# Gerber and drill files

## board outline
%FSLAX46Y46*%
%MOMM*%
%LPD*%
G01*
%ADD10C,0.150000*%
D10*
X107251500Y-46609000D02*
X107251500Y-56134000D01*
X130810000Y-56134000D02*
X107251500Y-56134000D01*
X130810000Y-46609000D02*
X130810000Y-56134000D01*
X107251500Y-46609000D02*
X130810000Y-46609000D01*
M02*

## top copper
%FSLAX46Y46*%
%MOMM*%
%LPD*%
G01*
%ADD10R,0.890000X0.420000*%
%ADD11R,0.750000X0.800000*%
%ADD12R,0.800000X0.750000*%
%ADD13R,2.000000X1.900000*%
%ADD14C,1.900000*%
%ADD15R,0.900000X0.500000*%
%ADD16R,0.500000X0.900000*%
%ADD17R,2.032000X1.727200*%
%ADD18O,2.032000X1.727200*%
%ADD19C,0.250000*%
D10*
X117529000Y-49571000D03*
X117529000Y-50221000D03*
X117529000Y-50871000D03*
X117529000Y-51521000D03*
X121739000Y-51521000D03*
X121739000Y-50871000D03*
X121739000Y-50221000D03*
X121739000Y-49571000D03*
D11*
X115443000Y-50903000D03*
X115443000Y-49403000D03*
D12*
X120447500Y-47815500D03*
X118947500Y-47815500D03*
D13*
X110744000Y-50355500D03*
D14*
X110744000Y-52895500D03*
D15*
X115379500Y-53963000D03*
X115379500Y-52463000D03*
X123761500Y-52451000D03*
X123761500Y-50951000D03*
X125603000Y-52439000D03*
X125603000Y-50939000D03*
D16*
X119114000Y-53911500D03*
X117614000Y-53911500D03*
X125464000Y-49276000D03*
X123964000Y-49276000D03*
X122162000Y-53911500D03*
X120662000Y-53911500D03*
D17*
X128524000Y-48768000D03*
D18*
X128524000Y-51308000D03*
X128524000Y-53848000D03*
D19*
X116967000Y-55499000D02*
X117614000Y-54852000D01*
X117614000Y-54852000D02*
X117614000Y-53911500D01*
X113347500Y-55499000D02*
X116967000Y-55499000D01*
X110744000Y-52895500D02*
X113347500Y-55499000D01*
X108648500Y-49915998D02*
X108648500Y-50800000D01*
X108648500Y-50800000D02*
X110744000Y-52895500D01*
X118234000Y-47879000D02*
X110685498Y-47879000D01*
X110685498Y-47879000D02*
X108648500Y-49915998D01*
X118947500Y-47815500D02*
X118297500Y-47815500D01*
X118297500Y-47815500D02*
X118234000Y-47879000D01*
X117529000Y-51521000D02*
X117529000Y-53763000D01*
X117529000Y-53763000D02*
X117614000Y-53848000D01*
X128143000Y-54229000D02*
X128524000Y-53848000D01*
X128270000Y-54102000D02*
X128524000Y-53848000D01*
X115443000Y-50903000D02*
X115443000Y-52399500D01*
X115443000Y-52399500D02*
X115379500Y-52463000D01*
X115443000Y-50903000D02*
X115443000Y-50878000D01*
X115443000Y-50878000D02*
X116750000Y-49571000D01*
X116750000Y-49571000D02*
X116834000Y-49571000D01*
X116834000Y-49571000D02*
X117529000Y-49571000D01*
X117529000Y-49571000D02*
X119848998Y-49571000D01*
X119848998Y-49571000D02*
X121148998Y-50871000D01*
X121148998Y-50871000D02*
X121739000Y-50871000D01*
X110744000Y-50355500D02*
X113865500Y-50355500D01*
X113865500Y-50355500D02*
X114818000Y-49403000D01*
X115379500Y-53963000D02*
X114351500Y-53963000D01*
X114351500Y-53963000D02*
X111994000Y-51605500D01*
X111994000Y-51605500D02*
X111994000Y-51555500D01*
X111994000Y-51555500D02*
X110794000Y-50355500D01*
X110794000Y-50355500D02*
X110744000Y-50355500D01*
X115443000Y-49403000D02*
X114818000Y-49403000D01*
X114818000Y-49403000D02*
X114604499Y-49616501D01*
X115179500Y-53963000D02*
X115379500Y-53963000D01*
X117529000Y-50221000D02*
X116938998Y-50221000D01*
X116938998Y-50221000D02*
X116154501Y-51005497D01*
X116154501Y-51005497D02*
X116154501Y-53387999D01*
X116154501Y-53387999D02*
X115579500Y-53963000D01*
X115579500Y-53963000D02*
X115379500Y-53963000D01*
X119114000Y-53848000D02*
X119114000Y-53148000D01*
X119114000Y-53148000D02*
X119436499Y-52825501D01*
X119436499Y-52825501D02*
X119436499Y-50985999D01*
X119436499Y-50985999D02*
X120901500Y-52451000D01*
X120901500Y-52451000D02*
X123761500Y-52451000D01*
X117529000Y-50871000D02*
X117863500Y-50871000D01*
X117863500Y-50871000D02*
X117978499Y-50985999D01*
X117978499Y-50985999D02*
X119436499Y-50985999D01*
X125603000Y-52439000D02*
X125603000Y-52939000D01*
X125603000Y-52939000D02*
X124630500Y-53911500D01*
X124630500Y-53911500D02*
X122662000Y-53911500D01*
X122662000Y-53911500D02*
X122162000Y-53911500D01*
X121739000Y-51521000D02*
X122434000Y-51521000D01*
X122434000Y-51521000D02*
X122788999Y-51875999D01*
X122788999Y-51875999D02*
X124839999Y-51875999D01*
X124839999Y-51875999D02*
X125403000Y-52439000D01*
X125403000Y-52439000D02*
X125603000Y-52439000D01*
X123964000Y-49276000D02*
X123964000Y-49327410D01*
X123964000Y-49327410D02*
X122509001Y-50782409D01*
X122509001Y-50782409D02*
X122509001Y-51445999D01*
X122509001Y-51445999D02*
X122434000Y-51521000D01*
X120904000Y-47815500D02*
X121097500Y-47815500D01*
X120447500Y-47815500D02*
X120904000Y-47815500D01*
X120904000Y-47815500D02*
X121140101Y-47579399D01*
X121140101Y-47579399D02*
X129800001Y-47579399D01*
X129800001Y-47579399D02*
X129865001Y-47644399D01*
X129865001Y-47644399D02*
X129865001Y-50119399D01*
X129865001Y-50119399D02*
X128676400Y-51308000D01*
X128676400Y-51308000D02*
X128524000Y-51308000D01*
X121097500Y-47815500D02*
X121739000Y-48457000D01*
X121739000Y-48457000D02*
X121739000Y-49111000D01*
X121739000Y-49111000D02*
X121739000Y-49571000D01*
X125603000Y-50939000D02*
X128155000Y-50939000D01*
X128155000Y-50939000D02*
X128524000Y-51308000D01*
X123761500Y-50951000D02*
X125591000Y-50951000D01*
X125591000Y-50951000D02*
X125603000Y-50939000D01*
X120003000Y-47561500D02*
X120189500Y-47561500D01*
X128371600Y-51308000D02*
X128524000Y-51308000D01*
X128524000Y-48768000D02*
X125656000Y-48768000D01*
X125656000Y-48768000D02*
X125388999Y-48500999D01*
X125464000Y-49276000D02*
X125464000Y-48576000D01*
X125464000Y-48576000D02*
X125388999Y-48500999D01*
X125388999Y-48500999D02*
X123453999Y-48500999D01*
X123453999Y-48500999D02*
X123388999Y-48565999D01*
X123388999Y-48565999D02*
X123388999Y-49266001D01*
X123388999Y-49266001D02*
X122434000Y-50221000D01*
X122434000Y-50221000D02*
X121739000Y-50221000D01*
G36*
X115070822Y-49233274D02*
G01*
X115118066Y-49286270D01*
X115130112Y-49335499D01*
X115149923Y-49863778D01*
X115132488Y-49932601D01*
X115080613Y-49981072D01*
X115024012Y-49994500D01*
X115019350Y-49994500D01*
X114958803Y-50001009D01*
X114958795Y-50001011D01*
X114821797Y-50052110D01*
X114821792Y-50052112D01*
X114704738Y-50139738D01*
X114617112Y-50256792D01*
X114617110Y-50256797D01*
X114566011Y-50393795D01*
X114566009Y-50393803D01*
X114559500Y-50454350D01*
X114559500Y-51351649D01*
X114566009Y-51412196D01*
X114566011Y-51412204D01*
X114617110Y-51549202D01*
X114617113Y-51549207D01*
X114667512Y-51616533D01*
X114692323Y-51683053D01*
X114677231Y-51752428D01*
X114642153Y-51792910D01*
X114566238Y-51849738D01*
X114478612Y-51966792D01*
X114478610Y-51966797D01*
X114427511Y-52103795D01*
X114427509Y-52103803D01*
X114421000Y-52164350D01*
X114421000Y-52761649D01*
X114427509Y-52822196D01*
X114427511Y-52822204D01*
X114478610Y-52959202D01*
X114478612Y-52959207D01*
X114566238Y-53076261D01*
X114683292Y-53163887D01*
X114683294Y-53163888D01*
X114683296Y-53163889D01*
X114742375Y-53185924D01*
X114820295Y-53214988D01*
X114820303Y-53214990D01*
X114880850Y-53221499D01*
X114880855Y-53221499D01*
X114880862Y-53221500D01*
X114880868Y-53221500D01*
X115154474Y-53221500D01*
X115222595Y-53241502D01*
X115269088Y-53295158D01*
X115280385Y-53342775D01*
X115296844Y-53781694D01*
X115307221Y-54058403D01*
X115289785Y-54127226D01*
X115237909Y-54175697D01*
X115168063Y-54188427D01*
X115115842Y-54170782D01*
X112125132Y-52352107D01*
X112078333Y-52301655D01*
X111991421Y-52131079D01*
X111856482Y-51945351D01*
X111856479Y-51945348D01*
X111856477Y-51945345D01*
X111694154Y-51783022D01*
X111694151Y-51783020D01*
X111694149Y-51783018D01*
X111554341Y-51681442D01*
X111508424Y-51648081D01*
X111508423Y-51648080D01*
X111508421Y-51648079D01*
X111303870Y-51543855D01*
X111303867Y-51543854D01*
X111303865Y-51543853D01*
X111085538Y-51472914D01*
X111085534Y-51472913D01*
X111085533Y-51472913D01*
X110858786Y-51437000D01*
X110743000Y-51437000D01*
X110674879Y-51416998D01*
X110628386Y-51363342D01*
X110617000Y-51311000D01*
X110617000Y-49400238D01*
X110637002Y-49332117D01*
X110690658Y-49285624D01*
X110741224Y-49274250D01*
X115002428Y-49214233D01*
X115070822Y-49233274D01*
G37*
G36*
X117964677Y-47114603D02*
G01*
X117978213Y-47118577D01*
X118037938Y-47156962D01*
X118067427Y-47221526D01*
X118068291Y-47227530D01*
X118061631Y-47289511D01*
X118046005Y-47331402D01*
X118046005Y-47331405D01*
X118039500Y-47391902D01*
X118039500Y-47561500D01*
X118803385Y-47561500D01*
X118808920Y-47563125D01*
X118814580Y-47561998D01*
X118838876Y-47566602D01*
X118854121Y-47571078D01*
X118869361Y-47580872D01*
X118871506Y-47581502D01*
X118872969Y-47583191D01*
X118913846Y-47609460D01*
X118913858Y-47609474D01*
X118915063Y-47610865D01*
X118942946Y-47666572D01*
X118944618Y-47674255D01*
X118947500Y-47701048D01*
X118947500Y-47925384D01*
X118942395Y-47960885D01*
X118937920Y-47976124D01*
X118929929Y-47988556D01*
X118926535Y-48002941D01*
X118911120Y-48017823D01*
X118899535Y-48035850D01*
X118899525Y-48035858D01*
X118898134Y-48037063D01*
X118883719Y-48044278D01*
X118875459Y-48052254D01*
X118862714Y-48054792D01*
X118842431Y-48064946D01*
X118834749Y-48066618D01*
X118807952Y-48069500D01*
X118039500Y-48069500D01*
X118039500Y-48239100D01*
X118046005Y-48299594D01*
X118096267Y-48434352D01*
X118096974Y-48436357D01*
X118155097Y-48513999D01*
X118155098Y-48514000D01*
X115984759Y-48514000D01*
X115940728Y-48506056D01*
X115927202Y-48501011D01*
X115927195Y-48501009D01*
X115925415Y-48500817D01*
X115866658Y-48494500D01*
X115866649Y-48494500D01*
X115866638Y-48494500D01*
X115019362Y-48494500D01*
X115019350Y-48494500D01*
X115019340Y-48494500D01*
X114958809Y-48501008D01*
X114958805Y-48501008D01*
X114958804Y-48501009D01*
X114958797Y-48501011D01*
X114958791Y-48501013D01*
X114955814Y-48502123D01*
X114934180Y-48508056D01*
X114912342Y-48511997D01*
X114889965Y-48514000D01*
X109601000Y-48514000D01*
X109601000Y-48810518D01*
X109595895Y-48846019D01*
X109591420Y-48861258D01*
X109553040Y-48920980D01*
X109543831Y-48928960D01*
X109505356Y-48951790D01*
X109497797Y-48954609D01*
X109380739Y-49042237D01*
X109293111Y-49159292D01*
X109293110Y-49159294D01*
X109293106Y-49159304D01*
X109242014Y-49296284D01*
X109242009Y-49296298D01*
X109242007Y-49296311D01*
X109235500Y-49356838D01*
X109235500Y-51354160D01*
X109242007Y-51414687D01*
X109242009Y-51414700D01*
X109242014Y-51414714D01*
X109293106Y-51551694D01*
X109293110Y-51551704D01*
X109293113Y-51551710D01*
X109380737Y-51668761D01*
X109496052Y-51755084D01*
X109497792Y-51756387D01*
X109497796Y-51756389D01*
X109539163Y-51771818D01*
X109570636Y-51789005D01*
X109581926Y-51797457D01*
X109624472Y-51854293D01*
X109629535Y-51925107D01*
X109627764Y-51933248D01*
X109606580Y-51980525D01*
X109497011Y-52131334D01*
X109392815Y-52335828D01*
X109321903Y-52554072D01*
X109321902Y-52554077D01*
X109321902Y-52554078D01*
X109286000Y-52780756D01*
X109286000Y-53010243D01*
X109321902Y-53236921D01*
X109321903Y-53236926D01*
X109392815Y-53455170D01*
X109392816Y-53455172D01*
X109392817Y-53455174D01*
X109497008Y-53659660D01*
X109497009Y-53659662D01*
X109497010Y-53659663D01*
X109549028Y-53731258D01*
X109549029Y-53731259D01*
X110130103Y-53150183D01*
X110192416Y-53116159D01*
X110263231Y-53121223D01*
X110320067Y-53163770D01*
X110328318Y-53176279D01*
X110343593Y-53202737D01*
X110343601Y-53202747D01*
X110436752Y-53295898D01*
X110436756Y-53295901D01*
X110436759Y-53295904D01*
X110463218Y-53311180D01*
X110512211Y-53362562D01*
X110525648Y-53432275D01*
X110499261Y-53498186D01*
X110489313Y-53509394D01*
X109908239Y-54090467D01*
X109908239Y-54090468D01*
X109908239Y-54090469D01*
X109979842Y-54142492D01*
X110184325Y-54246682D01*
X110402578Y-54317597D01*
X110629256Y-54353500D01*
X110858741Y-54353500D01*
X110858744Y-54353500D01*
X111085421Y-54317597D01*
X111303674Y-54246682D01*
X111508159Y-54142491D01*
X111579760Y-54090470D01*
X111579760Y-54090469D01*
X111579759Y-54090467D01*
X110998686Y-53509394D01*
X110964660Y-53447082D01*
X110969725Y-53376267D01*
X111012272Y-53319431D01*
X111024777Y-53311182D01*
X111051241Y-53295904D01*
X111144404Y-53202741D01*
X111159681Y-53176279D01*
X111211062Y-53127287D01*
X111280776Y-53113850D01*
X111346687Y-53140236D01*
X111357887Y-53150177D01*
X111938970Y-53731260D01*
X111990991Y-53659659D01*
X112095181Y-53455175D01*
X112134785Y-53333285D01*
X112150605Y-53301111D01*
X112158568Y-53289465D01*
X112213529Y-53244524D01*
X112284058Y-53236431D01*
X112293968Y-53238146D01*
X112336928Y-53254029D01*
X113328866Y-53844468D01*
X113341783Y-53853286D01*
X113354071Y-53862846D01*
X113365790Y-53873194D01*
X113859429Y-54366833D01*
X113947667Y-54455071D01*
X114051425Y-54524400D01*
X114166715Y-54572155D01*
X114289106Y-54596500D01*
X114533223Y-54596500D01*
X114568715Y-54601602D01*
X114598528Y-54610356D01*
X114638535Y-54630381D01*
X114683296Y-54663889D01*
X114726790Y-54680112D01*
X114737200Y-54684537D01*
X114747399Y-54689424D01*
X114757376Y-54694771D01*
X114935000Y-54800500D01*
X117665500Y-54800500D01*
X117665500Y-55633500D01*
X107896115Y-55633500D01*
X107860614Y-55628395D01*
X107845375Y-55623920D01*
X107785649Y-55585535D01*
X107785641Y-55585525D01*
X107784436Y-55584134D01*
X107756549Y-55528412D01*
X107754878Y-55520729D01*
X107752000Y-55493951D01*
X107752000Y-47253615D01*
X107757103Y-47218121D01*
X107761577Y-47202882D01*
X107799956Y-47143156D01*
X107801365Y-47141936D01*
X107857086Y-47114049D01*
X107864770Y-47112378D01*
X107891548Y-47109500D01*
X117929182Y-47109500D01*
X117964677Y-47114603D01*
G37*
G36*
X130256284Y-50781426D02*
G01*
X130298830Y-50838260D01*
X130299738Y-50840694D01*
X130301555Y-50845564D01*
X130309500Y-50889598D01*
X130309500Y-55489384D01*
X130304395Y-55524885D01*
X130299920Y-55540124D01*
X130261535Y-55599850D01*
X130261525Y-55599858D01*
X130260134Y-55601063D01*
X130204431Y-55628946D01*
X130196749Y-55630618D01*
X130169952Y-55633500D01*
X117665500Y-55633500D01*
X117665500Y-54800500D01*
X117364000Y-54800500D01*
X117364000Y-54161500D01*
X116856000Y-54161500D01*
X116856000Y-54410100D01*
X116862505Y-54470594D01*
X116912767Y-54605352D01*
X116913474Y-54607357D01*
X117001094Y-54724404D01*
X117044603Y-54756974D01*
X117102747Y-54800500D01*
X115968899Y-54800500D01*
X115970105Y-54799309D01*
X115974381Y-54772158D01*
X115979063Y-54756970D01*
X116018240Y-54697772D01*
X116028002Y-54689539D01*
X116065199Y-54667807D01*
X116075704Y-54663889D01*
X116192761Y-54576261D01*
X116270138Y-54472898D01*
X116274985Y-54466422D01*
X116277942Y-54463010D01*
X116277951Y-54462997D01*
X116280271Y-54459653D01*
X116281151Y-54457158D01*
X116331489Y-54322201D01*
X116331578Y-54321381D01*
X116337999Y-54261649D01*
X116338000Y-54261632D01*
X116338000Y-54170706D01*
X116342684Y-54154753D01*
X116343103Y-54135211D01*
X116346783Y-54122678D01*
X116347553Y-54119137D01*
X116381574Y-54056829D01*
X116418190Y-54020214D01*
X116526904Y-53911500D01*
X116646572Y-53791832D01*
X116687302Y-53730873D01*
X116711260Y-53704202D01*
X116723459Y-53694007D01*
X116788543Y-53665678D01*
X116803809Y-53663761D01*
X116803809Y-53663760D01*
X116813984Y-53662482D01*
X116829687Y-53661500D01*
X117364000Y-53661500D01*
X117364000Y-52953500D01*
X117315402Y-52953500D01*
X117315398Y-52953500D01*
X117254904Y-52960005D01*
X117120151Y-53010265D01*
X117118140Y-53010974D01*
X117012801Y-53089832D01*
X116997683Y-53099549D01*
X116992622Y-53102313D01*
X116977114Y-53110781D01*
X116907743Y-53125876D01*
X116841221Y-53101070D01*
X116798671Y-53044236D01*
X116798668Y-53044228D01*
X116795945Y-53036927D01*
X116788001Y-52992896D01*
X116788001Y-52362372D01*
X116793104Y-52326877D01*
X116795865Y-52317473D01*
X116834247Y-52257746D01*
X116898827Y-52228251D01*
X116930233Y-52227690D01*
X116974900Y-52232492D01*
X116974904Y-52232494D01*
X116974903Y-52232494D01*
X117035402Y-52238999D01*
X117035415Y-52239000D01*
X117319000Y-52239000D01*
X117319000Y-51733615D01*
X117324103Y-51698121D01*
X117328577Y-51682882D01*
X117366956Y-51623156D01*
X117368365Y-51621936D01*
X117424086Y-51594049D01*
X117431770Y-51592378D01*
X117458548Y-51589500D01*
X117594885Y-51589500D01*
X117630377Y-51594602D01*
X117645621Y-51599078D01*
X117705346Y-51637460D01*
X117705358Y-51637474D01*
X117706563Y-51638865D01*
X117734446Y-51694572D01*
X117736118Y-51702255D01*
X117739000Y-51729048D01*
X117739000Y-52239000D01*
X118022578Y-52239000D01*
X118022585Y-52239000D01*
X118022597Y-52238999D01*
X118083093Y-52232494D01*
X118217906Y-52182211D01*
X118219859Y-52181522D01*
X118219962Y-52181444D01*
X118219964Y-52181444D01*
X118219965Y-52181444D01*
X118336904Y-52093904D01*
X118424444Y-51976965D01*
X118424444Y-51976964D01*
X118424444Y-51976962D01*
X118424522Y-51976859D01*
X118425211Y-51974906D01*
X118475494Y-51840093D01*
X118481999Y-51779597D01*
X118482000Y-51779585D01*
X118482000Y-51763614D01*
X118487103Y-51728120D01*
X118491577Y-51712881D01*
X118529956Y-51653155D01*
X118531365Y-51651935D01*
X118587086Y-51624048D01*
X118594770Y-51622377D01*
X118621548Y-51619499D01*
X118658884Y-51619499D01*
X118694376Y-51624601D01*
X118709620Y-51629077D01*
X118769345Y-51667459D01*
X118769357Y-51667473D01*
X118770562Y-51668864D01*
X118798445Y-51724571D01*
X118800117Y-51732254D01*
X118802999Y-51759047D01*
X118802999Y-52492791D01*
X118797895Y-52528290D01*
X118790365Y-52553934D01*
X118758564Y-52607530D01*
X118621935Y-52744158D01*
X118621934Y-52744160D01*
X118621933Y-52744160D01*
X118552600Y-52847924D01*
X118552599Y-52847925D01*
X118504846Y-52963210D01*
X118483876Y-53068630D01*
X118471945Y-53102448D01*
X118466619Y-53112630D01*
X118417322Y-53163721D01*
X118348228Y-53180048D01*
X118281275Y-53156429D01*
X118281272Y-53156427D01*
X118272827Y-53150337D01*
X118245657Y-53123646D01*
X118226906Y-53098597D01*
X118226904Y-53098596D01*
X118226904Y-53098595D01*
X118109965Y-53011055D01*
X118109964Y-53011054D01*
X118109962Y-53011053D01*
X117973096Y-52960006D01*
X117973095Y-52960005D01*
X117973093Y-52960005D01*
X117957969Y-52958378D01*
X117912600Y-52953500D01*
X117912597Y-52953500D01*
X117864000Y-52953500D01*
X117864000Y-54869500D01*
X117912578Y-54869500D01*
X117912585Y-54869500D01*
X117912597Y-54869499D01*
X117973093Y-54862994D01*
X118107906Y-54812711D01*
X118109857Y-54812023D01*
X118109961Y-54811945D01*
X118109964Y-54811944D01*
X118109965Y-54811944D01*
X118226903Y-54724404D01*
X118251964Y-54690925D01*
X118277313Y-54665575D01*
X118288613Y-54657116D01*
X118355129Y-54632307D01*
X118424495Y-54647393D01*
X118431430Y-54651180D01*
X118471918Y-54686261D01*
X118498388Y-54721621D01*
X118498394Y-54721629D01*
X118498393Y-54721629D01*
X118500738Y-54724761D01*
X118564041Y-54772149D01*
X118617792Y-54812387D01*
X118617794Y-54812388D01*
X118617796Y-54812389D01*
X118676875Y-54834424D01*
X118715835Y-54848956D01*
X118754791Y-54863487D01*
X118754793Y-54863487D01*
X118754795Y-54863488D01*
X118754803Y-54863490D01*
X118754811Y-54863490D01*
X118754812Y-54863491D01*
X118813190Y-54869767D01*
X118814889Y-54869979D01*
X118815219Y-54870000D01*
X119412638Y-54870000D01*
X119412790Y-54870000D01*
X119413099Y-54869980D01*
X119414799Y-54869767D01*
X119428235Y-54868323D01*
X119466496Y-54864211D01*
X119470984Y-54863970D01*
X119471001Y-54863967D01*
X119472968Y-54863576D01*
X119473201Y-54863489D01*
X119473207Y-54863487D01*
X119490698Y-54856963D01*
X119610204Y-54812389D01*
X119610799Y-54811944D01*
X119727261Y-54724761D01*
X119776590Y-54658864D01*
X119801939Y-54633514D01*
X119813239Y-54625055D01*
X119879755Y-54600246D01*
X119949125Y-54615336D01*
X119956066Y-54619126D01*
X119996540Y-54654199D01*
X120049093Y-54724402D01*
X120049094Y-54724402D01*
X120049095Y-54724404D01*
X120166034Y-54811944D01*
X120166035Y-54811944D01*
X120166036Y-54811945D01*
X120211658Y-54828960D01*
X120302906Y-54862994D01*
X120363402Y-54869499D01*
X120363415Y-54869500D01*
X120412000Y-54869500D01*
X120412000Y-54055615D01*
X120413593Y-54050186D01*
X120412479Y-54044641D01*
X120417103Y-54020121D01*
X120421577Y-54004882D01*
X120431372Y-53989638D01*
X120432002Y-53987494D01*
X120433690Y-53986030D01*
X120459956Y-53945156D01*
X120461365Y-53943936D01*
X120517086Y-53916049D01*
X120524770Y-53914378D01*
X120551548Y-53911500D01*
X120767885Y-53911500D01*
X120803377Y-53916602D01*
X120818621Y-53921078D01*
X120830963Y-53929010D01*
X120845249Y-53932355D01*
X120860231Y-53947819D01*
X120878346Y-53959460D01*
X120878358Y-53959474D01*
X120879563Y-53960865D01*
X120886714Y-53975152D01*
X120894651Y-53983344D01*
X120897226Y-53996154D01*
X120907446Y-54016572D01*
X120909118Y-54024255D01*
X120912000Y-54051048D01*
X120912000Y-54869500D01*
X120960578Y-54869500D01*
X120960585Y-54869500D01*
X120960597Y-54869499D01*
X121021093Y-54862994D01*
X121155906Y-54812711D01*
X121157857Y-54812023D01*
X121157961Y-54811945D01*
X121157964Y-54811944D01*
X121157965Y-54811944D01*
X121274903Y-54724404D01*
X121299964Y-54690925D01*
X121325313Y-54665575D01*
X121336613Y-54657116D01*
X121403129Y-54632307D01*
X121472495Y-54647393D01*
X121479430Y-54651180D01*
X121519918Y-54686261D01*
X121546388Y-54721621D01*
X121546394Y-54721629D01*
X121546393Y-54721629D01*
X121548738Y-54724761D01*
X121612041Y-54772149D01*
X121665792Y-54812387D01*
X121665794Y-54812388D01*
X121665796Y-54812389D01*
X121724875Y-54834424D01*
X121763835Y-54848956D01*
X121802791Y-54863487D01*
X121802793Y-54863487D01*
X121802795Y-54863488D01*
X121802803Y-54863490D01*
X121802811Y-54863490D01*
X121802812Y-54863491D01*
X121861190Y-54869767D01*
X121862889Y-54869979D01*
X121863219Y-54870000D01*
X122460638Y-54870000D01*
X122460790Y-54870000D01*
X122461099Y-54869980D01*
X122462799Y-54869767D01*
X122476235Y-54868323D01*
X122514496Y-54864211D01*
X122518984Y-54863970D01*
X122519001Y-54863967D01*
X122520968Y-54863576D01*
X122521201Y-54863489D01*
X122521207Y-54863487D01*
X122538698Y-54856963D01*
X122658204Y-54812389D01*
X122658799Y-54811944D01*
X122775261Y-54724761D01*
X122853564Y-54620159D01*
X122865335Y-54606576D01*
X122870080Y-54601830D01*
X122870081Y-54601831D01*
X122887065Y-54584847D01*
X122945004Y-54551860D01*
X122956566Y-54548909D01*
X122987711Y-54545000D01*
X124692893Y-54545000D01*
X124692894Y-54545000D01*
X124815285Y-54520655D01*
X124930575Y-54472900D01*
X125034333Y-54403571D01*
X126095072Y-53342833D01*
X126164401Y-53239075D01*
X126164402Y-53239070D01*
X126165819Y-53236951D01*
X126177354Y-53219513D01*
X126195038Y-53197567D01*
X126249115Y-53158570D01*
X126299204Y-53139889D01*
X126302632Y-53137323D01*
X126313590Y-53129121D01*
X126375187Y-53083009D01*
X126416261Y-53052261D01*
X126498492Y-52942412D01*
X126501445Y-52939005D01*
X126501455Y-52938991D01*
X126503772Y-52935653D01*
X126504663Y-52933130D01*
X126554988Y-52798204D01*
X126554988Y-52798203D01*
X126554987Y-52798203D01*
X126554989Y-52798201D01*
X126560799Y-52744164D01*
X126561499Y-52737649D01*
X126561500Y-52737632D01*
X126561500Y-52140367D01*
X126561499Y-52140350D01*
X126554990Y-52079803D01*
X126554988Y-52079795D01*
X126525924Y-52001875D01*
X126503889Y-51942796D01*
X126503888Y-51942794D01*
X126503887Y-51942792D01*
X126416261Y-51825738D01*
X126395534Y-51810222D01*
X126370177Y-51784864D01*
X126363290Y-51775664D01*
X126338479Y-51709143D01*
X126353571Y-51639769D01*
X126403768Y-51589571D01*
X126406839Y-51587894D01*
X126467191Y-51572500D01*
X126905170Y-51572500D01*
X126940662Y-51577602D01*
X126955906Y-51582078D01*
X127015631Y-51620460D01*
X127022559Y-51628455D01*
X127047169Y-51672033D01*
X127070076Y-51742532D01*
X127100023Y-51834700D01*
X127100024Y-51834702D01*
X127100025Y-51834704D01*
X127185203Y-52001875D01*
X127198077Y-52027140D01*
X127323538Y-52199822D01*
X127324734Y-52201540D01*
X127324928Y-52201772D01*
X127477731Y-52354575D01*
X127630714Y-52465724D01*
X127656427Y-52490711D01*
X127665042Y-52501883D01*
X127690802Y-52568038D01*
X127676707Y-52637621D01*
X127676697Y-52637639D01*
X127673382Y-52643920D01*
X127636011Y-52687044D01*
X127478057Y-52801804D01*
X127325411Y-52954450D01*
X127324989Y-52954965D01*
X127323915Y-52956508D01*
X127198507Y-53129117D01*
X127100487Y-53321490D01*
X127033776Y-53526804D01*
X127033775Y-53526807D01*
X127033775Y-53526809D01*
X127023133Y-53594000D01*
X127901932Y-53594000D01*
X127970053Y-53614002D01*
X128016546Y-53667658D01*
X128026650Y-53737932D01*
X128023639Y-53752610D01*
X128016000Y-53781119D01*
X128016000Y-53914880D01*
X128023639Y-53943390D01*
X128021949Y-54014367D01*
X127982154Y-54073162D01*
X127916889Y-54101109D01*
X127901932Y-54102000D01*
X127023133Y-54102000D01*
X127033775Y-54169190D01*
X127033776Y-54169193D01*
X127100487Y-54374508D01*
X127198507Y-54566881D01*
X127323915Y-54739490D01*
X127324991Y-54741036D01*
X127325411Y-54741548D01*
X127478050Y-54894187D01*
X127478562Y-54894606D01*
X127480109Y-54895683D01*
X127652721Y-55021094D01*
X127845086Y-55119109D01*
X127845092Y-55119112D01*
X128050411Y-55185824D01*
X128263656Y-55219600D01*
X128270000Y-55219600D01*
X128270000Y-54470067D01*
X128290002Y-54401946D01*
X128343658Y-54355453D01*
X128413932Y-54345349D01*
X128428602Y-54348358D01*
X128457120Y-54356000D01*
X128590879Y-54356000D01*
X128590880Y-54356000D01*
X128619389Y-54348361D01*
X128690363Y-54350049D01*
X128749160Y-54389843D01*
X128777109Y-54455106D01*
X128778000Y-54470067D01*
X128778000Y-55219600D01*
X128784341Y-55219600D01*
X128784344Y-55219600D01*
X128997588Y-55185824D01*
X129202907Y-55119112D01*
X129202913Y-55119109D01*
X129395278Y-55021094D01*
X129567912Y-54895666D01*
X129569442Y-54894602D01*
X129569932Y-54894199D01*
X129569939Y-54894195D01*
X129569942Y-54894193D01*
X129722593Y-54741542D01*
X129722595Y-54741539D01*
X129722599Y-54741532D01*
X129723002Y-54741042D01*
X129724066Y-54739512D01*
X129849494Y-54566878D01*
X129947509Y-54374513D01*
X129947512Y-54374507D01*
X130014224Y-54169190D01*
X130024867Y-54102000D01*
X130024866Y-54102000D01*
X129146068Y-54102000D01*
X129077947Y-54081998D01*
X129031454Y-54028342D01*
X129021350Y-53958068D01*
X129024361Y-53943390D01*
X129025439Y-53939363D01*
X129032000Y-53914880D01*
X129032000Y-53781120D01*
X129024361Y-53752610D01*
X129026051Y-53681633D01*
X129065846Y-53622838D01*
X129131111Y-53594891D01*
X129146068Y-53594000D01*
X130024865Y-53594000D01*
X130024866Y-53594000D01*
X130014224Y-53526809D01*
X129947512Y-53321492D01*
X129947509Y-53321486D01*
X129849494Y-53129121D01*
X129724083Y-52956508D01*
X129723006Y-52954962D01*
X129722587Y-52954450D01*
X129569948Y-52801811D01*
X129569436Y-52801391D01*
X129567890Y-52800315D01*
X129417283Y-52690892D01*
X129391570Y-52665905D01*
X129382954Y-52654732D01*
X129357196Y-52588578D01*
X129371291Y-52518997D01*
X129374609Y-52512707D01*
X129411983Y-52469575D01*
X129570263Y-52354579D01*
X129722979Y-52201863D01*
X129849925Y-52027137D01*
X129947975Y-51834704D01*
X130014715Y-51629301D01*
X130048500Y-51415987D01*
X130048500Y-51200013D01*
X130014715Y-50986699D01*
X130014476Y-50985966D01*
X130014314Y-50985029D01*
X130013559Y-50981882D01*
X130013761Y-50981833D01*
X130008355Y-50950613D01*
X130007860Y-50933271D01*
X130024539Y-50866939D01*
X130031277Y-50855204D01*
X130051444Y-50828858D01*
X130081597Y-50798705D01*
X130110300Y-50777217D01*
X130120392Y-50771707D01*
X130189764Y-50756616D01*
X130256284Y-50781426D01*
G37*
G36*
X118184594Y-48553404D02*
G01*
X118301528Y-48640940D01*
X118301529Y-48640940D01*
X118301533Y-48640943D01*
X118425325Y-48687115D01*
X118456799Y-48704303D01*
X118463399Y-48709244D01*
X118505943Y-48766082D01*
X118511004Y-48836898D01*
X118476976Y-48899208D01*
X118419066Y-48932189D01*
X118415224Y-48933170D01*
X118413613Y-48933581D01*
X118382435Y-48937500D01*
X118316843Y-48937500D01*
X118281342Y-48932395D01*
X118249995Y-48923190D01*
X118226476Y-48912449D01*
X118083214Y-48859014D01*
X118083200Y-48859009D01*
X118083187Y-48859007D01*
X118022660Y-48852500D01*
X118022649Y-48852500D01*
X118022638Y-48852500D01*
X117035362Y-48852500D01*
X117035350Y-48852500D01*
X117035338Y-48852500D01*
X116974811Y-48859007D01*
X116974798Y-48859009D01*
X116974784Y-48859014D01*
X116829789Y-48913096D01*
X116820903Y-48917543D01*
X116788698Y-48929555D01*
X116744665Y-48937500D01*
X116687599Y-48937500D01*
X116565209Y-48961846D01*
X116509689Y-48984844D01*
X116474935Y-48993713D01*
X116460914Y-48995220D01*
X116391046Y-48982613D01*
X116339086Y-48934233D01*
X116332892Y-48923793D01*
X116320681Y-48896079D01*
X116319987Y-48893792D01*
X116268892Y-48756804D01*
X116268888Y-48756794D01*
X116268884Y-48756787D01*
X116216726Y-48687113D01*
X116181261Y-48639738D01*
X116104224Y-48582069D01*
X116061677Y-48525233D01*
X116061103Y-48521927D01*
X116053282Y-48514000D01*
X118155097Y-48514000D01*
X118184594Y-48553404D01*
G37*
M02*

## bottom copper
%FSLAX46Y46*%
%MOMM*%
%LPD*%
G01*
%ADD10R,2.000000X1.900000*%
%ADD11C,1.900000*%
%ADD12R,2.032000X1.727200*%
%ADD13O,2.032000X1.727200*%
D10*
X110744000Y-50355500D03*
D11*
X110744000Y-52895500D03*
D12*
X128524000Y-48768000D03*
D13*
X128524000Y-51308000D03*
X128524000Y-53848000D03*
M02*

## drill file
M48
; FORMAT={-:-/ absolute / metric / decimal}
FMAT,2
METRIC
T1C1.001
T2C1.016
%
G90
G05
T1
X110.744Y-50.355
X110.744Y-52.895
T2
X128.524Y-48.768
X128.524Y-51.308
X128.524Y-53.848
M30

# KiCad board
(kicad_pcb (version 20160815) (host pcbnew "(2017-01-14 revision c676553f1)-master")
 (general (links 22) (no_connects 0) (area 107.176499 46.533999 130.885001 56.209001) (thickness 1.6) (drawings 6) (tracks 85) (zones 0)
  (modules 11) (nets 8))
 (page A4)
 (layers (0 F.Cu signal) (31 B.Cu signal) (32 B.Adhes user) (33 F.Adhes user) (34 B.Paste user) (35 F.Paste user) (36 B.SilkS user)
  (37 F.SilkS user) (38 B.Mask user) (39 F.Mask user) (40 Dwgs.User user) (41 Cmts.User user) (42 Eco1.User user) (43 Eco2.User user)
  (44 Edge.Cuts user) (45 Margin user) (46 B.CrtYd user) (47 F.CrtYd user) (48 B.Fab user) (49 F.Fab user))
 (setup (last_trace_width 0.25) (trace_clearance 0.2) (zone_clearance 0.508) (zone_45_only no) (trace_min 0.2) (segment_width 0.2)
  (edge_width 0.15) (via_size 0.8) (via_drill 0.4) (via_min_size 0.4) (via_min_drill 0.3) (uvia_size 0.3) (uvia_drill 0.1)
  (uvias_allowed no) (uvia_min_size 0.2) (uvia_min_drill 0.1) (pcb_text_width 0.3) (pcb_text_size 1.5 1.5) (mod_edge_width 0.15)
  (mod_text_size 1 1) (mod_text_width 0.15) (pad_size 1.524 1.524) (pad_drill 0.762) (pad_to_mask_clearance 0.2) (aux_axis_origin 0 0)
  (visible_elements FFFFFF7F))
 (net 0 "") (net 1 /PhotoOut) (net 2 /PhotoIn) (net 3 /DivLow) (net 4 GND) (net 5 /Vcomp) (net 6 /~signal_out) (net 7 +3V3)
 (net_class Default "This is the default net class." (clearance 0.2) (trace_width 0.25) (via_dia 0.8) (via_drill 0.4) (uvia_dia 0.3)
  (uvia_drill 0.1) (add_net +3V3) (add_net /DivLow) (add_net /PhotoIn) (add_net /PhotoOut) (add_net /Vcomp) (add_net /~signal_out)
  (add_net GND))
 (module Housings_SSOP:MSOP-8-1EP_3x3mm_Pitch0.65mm (layer F.Cu) (at 119.634 50.546)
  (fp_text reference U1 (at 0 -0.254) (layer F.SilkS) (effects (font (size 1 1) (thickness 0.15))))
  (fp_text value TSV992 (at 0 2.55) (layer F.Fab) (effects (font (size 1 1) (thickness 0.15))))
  (pad 1 smd rect (at -2.105 -0.975) (size 0.89 0.42) (layers F.Cu F.Paste F.Mask) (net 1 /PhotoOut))
  (pad 2 smd rect (at -2.105 -0.325) (size 0.89 0.42) (layers F.Cu F.Paste F.Mask) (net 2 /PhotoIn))
  (pad 3 smd rect (at -2.105 0.325) (size 0.89 0.42) (layers F.Cu F.Paste F.Mask) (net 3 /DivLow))
  (pad 4 smd rect (at -2.105 0.975) (size 0.89 0.42) (layers F.Cu F.Paste F.Mask) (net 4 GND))
  (pad 5 smd rect (at 2.105 0.975) (size 0.89 0.42) (layers F.Cu F.Paste F.Mask) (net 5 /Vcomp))
  (pad 6 smd rect (at 2.105 0.325) (size 0.89 0.42) (layers F.Cu F.Paste F.Mask) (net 1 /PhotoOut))
  (pad 7 smd rect (at 2.105 -0.325) (size 0.89 0.42) (layers F.Cu F.Paste F.Mask) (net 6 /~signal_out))
  (pad 8 smd rect (at 2.105 -0.975) (size 0.89 0.42) (layers F.Cu F.Paste F.Mask) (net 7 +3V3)))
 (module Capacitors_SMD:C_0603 (layer F.Cu) (at 115.443 50.153 90)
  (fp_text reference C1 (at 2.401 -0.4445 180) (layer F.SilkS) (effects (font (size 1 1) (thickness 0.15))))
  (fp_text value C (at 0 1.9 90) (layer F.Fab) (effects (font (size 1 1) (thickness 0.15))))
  (pad 1 smd rect (at -0.75 0 90) (size 0.8 0.75) (layers F.Cu F.Paste F.Mask) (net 1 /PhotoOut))
  (pad 2 smd rect (at 0.75 0 90) (size 0.8 0.75) (layers F.Cu F.Paste F.Mask) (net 2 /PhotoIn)))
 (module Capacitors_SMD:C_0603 (layer F.Cu) (at 119.6975 47.8155)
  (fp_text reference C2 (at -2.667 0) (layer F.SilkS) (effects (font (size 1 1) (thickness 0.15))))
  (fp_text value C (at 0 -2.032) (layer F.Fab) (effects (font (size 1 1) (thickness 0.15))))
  (pad 2 smd rect (at 0.75 0) (size 0.8 0.75) (layers F.Cu F.Paste F.Mask) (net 7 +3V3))
  (pad 1 smd rect (at -0.75 0) (size 0.8 0.75) (layers F.Cu F.Paste F.Mask) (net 4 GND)))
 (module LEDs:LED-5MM (layer F.Cu) (at 110.744 50.3555 270)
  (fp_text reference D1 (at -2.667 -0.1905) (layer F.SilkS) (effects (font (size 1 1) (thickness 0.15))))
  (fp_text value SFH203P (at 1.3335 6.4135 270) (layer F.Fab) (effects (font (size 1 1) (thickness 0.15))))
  (pad 1 thru_hole rect (at 0 0) (size 2 1.9) (drill 1.00076) (layers *.Cu *.Mask F.SilkS) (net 2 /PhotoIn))
  (pad 2 thru_hole circle (at 2.54 0 270) (size 1.9 1.9) (drill 1.00076) (layers *.Cu *.Mask F.SilkS) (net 4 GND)))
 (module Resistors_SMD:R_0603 (layer F.Cu) (at 115.3795 53.213 270)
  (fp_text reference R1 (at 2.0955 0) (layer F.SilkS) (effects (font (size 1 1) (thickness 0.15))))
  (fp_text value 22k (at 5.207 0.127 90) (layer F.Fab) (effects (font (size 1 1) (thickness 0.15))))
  (pad 2 smd rect (at 0.75 0 270) (size 0.5 0.9) (layers F.Cu F.Paste F.Mask) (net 2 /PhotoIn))
  (pad 1 smd rect (at -0.75 0 270) (size 0.5 0.9) (layers F.Cu F.Paste F.Mask) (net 1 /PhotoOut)))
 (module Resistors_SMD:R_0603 (layer F.Cu) (at 123.7615 51.701 270)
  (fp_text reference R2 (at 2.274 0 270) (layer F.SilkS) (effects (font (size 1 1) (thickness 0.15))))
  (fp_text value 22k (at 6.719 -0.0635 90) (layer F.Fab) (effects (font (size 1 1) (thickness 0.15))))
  (pad 2 smd rect (at 0.75 0 270) (size 0.5 0.9) (layers F.Cu F.Paste F.Mask) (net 3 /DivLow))
  (pad 1 smd rect (at -0.75 0 270) (size 0.5 0.9) (layers F.Cu F.Paste F.Mask) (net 7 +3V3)))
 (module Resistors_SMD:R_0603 (layer F.Cu) (at 125.603 51.689 270)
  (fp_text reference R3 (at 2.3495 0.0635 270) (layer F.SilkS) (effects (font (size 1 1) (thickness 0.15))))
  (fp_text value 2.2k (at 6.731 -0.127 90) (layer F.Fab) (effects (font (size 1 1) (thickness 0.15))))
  (pad 2 smd rect (at 0.75 0 270) (size 0.5 0.9) (layers F.Cu F.Paste F.Mask) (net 5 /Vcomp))
  (pad 1 smd rect (at -0.75 0 270) (size 0.5 0.9) (layers F.Cu F.Paste F.Mask) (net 7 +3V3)))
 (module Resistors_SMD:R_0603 (layer F.Cu) (at 118.364 53.9115 180)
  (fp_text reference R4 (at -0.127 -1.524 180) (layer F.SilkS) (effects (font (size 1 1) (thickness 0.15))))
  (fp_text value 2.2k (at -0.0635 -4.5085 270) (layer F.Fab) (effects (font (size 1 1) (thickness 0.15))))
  (pad 1 smd rect (at -0.75 0 180) (size 0.5 0.9) (layers F.Cu F.Paste F.Mask) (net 3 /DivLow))
  (pad 2 smd rect (at 0.75 0 180) (size 0.5 0.9) (layers F.Cu F.Paste F.Mask) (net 4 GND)))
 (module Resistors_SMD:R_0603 (layer F.Cu) (at 124.714 49.276 180)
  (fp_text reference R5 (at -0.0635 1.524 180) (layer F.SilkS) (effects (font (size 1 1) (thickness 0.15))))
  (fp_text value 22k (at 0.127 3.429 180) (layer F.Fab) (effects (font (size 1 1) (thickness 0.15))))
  (pad 1 smd rect (at -0.75 0 180) (size 0.5 0.9) (layers F.Cu F.Paste F.Mask) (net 6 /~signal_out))
  (pad 2 smd rect (at 0.75 0 180) (size 0.5 0.9) (layers F.Cu F.Paste F.Mask) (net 5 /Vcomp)))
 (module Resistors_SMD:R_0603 (layer F.Cu) (at 121.412 53.9115 180)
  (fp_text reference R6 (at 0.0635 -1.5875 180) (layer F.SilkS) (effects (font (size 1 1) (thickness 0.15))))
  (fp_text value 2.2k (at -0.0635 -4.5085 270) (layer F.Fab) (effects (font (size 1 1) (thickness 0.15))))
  (pad 1 smd rect (at -0.75 0 180) (size 0.5 0.9) (layers F.Cu F.Paste F.Mask) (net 5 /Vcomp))
  (pad 2 smd rect (at 0.75 0 180) (size 0.5 0.9) (layers F.Cu F.Paste F.Mask) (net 4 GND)))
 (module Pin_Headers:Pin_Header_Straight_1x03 (layer F.Cu) (at 128.524 48.768)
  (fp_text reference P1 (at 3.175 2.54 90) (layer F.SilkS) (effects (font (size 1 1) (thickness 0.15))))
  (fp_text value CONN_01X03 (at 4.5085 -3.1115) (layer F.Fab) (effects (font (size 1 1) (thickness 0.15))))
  (pad 1 thru_hole rect (at 0 0) (size 2.032 1.7272) (drill 1.016) (layers *.Cu *.Mask F.SilkS) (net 6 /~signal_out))
  (pad 2 thru_hole oval (at 0 2.54) (size 2.032 1.7272) (drill 1.016) (layers *.Cu *.Mask F.SilkS) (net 7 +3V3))
  (pad 3 thru_hole oval (at 0 5.08) (size 2.032 1.7272) (drill 1.016) (layers *.Cu *.Mask F.SilkS) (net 4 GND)))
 (gr_line (start 107.2515 46.609) (end 107.2515 56.134) (layer Edge.Cuts) (width 0.15))
 (gr_line (start 130.81 56.134) (end 107.2515 56.134) (layer Edge.Cuts) (width 0.15))
 (gr_line (start 130.81 46.609) (end 130.81 56.134) (layer Edge.Cuts) (width 0.15))
 (gr_line (start 107.2515 46.609) (end 130.81 46.609) (layer Edge.Cuts) (width 0.15))
 (segment (start 116.967 55.499) (end 117.614 54.852) (width 0.25) (layer F.Cu) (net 4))
 (segment (start 117.614 54.852) (end 117.614 53.9115) (width 0.25) (layer F.Cu) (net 4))
 (segment (start 113.3475 55.499) (end 116.967 55.499) (width 0.25) (layer F.Cu) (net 4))
 (segment (start 110.744 52.8955) (end 113.3475 55.499) (width 0.25) (layer F.Cu) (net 4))
 (segment (start 108.6485 49.915998) (end 108.6485 50.8) (width 0.25) (layer F.Cu) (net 4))
 (segment (start 108.6485 50.8) (end 110.744 52.8955) (width 0.25) (layer F.Cu) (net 4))
 (segment (start 118.234 47.879) (end 110.685498 47.879) (width 0.25) (layer F.Cu) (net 4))
 (segment (start 110.685498 47.879) (end 108.6485 49.915998) (width 0.25) (layer F.Cu) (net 4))
 (segment (start 118.9475 47.8155) (end 118.2975 47.8155) (width 0.25) (layer F.Cu) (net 4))
 (segment (start 118.2975 47.8155) (end 118.234 47.879) (width 0.25) (layer F.Cu) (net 4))
 (segment (start 117.529 51.521) (end 117.529 53.763) (width 0.25) (layer F.Cu) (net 4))
 (segment (start 117.529 53.763) (end 117.614 53.848) (width 0.25) (layer F.Cu) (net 4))
 (segment (start 128.143 54.229) (end 128.524 53.848) (width 0.25) (layer F.Cu) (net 4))
 (segment (start 128.27 54.102) (end 128.524 53.848) (width 0.25) (layer F.Cu) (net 4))
 (segment (start 115.443 50.903) (end 115.443 52.3995) (width 0.25) (layer F.Cu) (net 1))
 (segment (start 115.443 52.3995) (end 115.3795 52.463) (width 0.25) (layer F.Cu) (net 1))
 (segment (start 115.443 50.903) (end 115.443 50.878) (width 0.25) (layer F.Cu) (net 1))
 (segment (start 115.443 50.878) (end 116.75 49.571) (width 0.25) (layer F.Cu) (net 1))
 (segment (start 116.75 49.571) (end 116.834 49.571) (width 0.25) (layer F.Cu) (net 1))
 (segment (start 116.834 49.571) (end 117.529 49.571) (width 0.25) (layer F.Cu) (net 1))
 (segment (start 117.529 49.571) (end 119.848998 49.571) (width 0.25) (layer F.Cu) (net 1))
 (segment (start 119.848998 49.571) (end 121.148998 50.871) (width 0.25) (layer F.Cu) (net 1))
 (segment (start 121.148998 50.871) (end 121.739 50.871) (width 0.25) (layer F.Cu) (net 1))
 (segment (start 110.744 50.3555) (end 113.8655 50.3555) (width 0.25) (layer F.Cu) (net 2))
 (segment (start 113.8655 50.3555) (end 114.818 49.403) (width 0.25) (layer F.Cu) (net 2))
 (segment (start 115.3795 53.963) (end 114.3515 53.963) (width 0.25) (layer F.Cu) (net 2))
 (segment (start 114.3515 53.963) (end 111.994 51.6055) (width 0.25) (layer F.Cu) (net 2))
 (segment (start 111.994 51.6055) (end 111.994 51.5555) (width 0.25) (layer F.Cu) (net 2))
 (segment (start 111.994 51.5555) (end 110.794 50.3555) (width 0.25) (layer F.Cu) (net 2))
 (segment (start 110.794 50.3555) (end 110.744 50.3555) (width 0.25) (layer F.Cu) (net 2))
 (segment (start 115.443 49.403) (end 114.818 49.403) (width 0.25) (layer F.Cu) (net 2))
 (segment (start 114.818 49.403) (end 114.604499 49.616501) (width 0.25) (layer F.Cu) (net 2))
 (segment (start 115.1795 53.963) (end 115.3795 53.963) (width 0.25) (layer F.Cu) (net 2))
 (segment (start 117.529 50.221) (end 116.938998 50.221) (width 0.25) (layer F.Cu) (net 2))
 (segment (start 116.938998 50.221) (end 116.154501 51.005497) (width 0.25) (layer F.Cu) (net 2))
 (segment (start 116.154501 51.005497) (end 116.154501 53.387999) (width 0.25) (layer F.Cu) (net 2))
 (segment (start 116.154501 53.387999) (end 115.5795 53.963) (width 0.25) (layer F.Cu) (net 2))
 (segment (start 115.5795 53.963) (end 115.3795 53.963) (width 0.25) (layer F.Cu) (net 2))
 (segment (start 119.114 53.848) (end 119.114 53.148) (width 0.25) (layer F.Cu) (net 3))
 (segment (start 119.114 53.148) (end 119.436499 52.825501) (width 0.25) (layer F.Cu) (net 3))
 (segment (start 119.436499 52.825501) (end 119.436499 50.985999) (width 0.25) (layer F.Cu) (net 3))
 (segment (start 119.436499 50.985999) (end 120.9015 52.451) (width 0.25) (layer F.Cu) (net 3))
 (segment (start 120.9015 52.451) (end 123.7615 52.451) (width 0.25) (layer F.Cu) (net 3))
 (segment (start 117.529 50.871) (end 117.8635 50.871) (width 0.25) (layer F.Cu) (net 3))
 (segment (start 117.8635 50.871) (end 117.978499 50.985999) (width 0.25) (layer F.Cu) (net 3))
 (segment (start 117.978499 50.985999) (end 119.436499 50.985999) (width 0.25) (layer F.Cu) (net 3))
 (segment (start 125.603 52.439) (end 125.603 52.939) (width 0.25) (layer F.Cu) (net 5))
 (segment (start 125.603 52.939) (end 124.6305 53.9115) (width 0.25) (layer F.Cu) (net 5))
 (segment (start 124.6305 53.9115) (end 122.662 53.9115) (width 0.25) (layer F.Cu) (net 5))
 (segment (start 122.662 53.9115) (end 122.162 53.9115) (width 0.25) (layer F.Cu) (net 5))
 (segment (start 121.739 51.521) (end 122.434 51.521) (width 0.25) (layer F.Cu) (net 5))
 (segment (start 122.434 51.521) (end 122.788999 51.875999) (width 0.25) (layer F.Cu) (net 5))
 (segment (start 122.788999 51.875999) (end 124.839999 51.875999) (width 0.25) (layer F.Cu) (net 5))
 (segment (start 124.839999 51.875999) (end 125.403 52.439) (width 0.25) (layer F.Cu) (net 5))
 (segment (start 125.403 52.439) (end 125.603 52.439) (width 0.25) (layer F.Cu) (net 5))
 (segment (start 123.964 49.276) (end 123.964 49.32741) (width 0.25) (layer F.Cu) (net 5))
 (segment (start 123.964 49.32741) (end 122.509001 50.782409) (width 0.25) (layer F.Cu) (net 5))
 (segment (start 122.509001 50.782409) (end 122.509001 51.445999) (width 0.25) (layer F.Cu) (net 5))
 (segment (start 122.509001 51.445999) (end 122.434 51.521) (width 0.25) (layer F.Cu) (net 5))
 (segment (start 120.904 47.8155) (end 121.0975 47.8155) (width 0.25) (layer F.Cu) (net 7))
 (segment (start 120.4475 47.8155) (end 120.904 47.8155) (width 0.25) (layer F.Cu) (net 7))
 (segment (start 120.904 47.8155) (end 121.140101 47.579399) (width 0.25) (layer F.Cu) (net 7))
 (segment (start 121.140101 47.579399) (end 129.800001 47.579399) (width 0.25) (layer F.Cu) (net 7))
 (segment (start 129.800001 47.579399) (end 129.865001 47.644399) (width 0.25) (layer F.Cu) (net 7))
 (segment (start 129.865001 47.644399) (end 129.865001 50.119399) (width 0.25) (layer F.Cu) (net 7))
 (segment (start 129.865001 50.119399) (end 128.6764 51.308) (width 0.25) (layer F.Cu) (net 7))
 (segment (start 128.6764 51.308) (end 128.524 51.308) (width 0.25) (layer F.Cu) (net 7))
 (segment (start 121.0975 47.8155) (end 121.739 48.457) (width 0.25) (layer F.Cu) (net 7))
 (segment (start 121.739 48.457) (end 121.739 49.111) (width 0.25) (layer F.Cu) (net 7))
 (segment (start 121.739 49.111) (end 121.739 49.571) (width 0.25) (layer F.Cu) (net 7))
 (segment (start 125.603 50.939) (end 128.155 50.939) (width 0.25) (layer F.Cu) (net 7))
 (segment (start 128.155 50.939) (end 128.524 51.308) (width 0.25) (layer F.Cu) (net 7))
 (segment (start 123.7615 50.951) (end 125.591 50.951) (width 0.25) (layer F.Cu) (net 7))
 (segment (start 125.591 50.951) (end 125.603 50.939) (width 0.25) (layer F.Cu) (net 7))
 (segment (start 120.003 47.5615) (end 120.1895 47.5615) (width 0.25) (layer F.Cu) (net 7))
 (segment (start 128.3716 51.308) (end 128.524 51.308) (width 0.25) (layer F.Cu) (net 7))
 (segment (start 128.524 48.768) (end 125.656 48.768) (width 0.25) (layer F.Cu) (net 6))
 (segment (start 125.656 48.768) (end 125.388999 48.500999) (width 0.25) (layer F.Cu) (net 6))
 (segment (start 125.464 49.276) (end 125.464 48.576) (width 0.25) (layer F.Cu) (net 6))
 (segment (start 125.464 48.576) (end 125.388999 48.500999) (width 0.25) (layer F.Cu) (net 6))
 (segment (start 125.388999 48.500999) (end 123.453999 48.500999) (width 0.25) (layer F.Cu) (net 6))
 (segment (start 123.453999 48.500999) (end 123.388999 48.565999) (width 0.25) (layer F.Cu) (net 6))
 (segment (start 123.388999 48.565999) (end 123.388999 49.266001) (width 0.25) (layer F.Cu) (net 6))
 (segment (start 123.388999 49.266001) (end 122.434 50.221) (width 0.25) (layer F.Cu) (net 6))
 (segment (start 122.434 50.221) (end 121.739 50.221) (width 0.25) (layer F.Cu) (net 6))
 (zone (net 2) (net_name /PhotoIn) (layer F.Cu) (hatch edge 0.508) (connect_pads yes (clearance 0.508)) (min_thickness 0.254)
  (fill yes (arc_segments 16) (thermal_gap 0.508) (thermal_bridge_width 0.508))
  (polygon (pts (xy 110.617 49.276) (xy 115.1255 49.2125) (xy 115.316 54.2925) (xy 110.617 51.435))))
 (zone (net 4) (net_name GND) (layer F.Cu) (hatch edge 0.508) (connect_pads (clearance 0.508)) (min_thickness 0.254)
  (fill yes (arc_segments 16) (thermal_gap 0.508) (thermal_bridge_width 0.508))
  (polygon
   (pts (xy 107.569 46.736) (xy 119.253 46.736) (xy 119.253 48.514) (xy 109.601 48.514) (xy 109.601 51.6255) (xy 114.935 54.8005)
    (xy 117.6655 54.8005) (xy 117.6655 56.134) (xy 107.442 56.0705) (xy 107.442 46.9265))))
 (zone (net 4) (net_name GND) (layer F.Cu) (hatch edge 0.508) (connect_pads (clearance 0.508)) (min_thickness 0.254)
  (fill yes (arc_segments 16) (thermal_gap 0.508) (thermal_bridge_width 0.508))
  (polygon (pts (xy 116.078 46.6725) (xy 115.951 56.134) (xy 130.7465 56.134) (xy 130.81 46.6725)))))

